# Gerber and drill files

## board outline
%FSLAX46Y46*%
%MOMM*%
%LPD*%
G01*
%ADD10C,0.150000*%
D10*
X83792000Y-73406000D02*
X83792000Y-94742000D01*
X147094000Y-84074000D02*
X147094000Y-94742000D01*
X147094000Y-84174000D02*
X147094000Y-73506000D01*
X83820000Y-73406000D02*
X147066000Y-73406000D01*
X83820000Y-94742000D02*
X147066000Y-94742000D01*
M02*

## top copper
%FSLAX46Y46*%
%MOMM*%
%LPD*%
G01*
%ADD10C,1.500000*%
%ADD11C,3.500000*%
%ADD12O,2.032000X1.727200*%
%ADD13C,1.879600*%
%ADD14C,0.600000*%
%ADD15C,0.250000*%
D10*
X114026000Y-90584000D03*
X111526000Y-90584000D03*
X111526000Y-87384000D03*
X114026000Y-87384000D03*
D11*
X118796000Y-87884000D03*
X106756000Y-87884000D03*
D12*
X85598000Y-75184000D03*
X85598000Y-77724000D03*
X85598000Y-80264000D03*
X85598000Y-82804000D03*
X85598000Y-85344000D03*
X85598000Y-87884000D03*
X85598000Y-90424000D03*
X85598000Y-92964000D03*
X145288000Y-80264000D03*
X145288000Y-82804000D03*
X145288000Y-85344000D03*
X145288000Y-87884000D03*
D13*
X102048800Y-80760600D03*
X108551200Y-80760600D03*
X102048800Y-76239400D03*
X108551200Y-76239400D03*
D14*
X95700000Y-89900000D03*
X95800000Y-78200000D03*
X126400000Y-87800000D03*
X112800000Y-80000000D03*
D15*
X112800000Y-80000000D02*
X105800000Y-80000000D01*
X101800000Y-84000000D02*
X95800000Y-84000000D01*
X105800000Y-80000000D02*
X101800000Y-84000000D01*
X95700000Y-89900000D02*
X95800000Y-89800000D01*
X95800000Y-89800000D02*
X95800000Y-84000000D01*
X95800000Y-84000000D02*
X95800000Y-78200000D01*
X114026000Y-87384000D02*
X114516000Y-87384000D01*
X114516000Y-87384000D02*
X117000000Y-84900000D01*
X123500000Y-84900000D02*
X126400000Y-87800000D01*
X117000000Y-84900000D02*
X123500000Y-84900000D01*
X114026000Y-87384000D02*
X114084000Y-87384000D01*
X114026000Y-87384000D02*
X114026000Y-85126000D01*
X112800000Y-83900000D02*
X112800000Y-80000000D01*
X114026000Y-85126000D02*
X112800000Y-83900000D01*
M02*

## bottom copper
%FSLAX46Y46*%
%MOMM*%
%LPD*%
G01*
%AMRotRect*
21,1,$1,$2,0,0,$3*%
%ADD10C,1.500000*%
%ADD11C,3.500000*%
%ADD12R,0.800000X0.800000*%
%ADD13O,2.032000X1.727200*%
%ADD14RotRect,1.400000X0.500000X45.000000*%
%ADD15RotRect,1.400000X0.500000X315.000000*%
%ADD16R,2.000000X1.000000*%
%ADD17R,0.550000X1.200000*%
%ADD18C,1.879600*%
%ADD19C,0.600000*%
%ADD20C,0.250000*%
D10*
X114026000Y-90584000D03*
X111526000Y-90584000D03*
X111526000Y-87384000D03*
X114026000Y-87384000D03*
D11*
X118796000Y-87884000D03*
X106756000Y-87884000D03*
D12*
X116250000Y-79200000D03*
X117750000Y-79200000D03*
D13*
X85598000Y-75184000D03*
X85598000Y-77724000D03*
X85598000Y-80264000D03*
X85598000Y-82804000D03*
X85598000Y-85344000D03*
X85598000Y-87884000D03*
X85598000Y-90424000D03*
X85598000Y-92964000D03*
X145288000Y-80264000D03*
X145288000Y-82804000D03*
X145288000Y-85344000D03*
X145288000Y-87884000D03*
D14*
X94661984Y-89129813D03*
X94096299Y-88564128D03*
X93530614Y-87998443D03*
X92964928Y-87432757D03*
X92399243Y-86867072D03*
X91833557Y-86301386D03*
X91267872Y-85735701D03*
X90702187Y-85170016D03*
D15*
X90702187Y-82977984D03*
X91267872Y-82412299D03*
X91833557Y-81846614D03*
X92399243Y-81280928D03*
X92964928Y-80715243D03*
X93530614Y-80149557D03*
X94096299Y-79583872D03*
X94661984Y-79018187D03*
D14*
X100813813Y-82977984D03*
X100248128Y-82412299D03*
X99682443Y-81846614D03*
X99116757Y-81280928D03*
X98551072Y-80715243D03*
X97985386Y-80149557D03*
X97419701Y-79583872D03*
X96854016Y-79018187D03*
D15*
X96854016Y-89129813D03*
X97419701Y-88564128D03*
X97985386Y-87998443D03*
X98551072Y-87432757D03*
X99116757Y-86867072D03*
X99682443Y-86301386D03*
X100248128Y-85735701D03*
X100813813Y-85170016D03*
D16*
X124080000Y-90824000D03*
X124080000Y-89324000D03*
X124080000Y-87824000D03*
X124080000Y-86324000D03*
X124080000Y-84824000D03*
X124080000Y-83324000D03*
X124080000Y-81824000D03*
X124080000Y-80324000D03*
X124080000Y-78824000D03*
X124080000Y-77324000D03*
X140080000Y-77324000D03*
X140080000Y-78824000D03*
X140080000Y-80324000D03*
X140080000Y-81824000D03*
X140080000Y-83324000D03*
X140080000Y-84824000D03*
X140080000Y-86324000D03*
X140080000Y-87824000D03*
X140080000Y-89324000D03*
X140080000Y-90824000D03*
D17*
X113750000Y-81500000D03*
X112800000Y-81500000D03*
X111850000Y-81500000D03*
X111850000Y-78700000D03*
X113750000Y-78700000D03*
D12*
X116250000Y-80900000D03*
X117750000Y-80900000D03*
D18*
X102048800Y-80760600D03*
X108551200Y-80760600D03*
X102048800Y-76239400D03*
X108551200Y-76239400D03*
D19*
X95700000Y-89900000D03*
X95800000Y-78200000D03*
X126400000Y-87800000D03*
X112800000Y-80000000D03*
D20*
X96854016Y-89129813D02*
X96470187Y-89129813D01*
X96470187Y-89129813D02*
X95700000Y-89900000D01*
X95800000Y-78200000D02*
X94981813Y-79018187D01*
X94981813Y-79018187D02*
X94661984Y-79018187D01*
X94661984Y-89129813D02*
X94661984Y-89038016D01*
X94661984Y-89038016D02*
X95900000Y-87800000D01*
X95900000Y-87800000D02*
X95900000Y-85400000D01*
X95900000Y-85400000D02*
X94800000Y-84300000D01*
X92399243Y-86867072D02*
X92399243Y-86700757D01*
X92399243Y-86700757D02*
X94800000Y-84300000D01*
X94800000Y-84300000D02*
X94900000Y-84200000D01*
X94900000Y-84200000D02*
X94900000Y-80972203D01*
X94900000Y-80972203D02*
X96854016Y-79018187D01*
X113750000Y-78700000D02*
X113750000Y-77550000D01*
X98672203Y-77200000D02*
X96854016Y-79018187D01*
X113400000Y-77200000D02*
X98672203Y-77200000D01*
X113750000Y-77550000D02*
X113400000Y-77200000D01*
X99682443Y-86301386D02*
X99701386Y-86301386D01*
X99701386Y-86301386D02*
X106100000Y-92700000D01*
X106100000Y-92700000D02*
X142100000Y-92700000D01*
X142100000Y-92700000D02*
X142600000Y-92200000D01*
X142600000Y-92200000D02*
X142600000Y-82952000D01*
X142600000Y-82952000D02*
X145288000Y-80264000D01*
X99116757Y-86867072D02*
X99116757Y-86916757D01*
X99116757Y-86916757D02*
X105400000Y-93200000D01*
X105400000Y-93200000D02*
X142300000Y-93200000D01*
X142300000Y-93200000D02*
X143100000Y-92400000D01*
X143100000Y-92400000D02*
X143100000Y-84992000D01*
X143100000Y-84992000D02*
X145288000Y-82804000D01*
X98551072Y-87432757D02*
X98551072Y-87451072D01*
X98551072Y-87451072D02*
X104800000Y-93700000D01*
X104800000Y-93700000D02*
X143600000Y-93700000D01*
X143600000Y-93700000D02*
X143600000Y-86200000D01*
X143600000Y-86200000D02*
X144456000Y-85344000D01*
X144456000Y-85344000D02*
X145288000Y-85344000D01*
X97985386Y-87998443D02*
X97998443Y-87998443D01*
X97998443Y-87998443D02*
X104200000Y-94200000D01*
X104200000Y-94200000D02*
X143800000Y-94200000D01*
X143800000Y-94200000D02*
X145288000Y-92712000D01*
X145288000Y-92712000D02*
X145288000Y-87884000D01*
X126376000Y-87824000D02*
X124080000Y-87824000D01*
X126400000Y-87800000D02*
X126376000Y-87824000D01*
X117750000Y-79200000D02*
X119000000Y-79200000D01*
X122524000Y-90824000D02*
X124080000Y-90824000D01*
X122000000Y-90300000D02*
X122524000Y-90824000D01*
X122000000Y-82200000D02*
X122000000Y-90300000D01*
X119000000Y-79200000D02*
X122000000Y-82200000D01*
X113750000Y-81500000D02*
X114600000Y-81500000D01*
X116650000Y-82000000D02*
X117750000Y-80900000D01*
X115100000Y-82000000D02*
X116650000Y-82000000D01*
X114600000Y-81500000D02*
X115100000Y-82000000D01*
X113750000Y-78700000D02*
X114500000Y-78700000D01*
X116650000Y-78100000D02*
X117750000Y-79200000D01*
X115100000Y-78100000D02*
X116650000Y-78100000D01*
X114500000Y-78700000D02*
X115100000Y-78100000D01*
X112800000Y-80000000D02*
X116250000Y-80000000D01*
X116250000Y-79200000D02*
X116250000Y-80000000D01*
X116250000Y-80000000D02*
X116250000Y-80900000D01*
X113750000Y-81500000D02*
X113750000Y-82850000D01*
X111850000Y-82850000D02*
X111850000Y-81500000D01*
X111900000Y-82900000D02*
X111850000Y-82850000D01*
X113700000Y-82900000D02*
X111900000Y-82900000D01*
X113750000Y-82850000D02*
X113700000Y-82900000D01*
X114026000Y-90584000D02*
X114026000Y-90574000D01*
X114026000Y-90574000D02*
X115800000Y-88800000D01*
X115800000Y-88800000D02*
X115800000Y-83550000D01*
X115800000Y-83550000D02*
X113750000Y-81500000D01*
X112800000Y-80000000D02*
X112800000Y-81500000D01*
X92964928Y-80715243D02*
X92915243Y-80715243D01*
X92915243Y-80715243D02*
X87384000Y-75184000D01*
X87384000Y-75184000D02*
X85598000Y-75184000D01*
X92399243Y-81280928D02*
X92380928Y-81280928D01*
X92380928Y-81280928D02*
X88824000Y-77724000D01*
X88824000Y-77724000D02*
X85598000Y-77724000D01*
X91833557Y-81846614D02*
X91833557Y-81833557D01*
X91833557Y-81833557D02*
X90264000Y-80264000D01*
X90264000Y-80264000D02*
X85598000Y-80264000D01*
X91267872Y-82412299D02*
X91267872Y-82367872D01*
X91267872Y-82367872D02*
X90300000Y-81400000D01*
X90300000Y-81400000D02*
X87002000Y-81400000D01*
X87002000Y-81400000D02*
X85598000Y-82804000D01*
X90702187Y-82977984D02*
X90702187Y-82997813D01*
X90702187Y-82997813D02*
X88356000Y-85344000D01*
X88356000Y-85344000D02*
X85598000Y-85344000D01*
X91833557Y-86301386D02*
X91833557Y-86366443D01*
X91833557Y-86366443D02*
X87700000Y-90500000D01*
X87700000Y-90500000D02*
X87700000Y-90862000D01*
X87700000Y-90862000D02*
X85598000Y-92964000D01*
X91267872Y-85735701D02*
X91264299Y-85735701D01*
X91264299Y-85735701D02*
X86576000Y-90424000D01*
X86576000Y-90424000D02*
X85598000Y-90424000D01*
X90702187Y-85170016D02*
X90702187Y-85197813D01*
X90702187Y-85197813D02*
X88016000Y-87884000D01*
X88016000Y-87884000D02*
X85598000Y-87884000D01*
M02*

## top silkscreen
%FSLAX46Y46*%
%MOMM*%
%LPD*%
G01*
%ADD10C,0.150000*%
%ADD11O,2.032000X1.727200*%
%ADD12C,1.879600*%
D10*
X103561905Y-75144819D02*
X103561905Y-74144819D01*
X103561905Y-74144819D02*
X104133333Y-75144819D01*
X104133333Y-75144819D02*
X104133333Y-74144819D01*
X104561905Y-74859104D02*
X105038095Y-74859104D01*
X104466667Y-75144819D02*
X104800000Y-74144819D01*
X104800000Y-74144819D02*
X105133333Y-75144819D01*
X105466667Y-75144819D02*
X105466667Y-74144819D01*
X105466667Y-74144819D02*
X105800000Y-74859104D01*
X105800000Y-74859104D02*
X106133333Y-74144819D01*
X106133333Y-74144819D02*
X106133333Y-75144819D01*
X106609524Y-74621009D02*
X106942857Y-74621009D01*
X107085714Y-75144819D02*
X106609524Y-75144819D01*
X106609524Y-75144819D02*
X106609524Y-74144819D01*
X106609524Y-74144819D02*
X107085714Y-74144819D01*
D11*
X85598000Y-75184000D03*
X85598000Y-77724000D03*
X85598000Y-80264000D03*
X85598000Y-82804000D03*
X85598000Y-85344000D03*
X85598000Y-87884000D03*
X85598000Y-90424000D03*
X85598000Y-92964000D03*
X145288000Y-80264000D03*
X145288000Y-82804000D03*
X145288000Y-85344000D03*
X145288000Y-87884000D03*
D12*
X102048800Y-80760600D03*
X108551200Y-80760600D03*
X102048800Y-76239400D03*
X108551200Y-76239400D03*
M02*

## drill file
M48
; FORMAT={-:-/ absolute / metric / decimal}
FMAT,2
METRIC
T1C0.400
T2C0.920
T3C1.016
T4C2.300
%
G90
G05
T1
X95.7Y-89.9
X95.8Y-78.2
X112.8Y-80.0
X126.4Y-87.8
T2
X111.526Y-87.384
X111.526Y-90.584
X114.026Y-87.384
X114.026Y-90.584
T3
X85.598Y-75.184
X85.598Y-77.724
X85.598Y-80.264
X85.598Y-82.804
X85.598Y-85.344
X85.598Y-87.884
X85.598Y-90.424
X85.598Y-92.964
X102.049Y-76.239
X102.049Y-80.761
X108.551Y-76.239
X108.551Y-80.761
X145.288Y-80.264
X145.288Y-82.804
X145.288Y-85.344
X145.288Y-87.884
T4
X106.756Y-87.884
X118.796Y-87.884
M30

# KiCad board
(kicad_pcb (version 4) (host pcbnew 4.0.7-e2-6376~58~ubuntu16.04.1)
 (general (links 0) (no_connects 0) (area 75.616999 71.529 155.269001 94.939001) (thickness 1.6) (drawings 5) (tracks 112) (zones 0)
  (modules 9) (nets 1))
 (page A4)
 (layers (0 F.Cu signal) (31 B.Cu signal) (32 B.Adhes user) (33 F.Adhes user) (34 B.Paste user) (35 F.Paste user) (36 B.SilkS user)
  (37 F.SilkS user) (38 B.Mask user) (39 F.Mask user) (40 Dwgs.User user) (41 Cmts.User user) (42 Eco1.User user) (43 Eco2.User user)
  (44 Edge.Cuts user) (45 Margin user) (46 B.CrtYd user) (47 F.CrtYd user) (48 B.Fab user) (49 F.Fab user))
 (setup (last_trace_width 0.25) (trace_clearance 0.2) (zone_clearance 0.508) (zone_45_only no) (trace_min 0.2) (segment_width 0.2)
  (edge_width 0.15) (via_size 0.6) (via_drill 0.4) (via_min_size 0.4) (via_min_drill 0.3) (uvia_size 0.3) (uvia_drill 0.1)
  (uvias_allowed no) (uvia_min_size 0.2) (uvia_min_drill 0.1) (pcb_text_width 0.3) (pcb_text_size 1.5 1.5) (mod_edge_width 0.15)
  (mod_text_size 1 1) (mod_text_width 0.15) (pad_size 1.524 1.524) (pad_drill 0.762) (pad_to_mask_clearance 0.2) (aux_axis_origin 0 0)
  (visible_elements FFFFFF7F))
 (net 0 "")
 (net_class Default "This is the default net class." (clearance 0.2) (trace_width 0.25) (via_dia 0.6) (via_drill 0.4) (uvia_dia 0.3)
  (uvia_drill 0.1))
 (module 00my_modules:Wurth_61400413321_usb (layer B.Cu) (at 112.776 87.884)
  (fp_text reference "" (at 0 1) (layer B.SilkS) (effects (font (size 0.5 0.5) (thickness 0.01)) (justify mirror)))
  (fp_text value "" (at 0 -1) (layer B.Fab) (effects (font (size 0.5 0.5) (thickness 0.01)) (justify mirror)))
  (pad V thru_hole circle (at 1.25 2.7) (size 1.5 1.5) (drill 0.92) (layers *.Cu *.Mask B.SilkS))
  (pad - thru_hole circle (at -1.25 2.7) (size 1.5 1.5) (drill 0.92) (layers *.Cu *.Mask B.SilkS))
  (pad + thru_hole circle (at -1.25 -0.5) (size 1.5 1.5) (drill 0.92) (layers *.Cu *.Mask B.SilkS))
  (pad G thru_hole circle (at 1.25 -0.5) (size 1.5 1.5) (drill 0.92) (layers *.Cu *.Mask B.SilkS))
  (pad X thru_hole circle (at 6.02 0) (size 3.5 3.5) (drill 2.3) (layers *.Cu *.Mask B.SilkS))
  (pad X thru_hole circle (at -6.02 0) (size 3.5 3.5) (drill 2.3) (layers *.Cu *.Mask B.SilkS)))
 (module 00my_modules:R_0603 (layer B.Cu) (at 117 79.2)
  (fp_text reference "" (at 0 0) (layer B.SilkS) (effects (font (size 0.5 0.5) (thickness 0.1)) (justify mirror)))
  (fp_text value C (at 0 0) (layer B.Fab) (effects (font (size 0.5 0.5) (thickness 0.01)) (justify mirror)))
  (pad 1 smd rect (at -0.75 0) (size 0.8 0.8) (layers B.Cu B.Paste B.Mask))
  (pad 2 smd rect (at 0.75 0) (size 0.8 0.8) (layers B.Cu B.Paste B.Mask)))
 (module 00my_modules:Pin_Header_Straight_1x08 (layer F.Cu) (at 85.598 75.184)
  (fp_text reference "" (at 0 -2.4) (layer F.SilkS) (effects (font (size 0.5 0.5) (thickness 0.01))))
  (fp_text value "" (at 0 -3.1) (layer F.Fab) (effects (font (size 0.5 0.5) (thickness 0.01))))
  (pad 1 thru_hole oval (at 0 0) (size 2.032 1.7272) (drill 1.016) (layers *.Cu *.Mask F.SilkS))
  (pad 2 thru_hole oval (at 0 2.54) (size 2.032 1.7272) (drill 1.016) (layers *.Cu *.Mask F.SilkS))
  (pad 3 thru_hole oval (at 0 5.08) (size 2.032 1.7272) (drill 1.016) (layers *.Cu *.Mask F.SilkS))
  (pad 4 thru_hole oval (at 0 7.62) (size 2.032 1.7272) (drill 1.016) (layers *.Cu *.Mask F.SilkS))
  (pad 5 thru_hole oval (at 0 10.16) (size 2.032 1.7272) (drill 1.016) (layers *.Cu *.Mask F.SilkS))
  (pad 6 thru_hole oval (at 0 12.7) (size 2.032 1.7272) (drill 1.016) (layers *.Cu *.Mask F.SilkS))
  (pad 7 thru_hole oval (at 0 15.24) (size 2.032 1.7272) (drill 1.016) (layers *.Cu *.Mask F.SilkS))
  (pad 8 thru_hole oval (at 0 17.78) (size 2.032 1.7272) (drill 1.016) (layers *.Cu *.Mask F.SilkS)))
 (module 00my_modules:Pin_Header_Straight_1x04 (layer F.Cu) (at 145.288 80.264)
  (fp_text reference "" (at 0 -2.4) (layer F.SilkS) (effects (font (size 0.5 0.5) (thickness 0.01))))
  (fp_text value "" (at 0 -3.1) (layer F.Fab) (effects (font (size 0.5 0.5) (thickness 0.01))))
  (pad 1 thru_hole oval (at 0 0) (size 2.032 1.7272) (drill 1.016) (layers *.Cu *.Mask F.SilkS))
  (pad 2 thru_hole oval (at 0 2.54) (size 2.032 1.7272) (drill 1.016) (layers *.Cu *.Mask F.SilkS))
  (pad 3 thru_hole oval (at 0 5.08) (size 2.032 1.7272) (drill 1.016) (layers *.Cu *.Mask F.SilkS))
  (pad 4 thru_hole oval (at 0 7.62) (size 2.032 1.7272) (drill 1.016) (layers *.Cu *.Mask F.SilkS)))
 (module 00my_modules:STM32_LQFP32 (layer B.Cu) (at 95.758 84.074 45)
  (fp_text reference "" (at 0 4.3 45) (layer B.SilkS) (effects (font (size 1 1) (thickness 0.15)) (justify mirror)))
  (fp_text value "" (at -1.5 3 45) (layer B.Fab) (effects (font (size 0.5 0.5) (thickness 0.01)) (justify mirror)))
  (pad 3.3 smd rect (at -4.35 2.8 45) (size 1.4 0.5) (layers B.Cu B.Paste B.Mask))
  (pad PF0 smd rect (at -4.35 2 45) (size 1.4 0.5) (layers B.Cu B.Paste B.Mask))
  (pad PF1 smd rect (at -4.35 1.2 45) (size 1.4 0.5) (layers B.Cu B.Paste B.Mask))
  (pad RST smd rect (at -4.35 0.4 45) (size 1.4 0.5) (layers B.Cu B.Paste B.Mask))
  (pad 3.3 smd rect (at -4.35 -0.4 45) (size 1.4 0.5) (layers B.Cu B.Paste B.Mask))
  (pad PA0 smd rect (at -4.35 -1.2 45) (size 1.4 0.5) (layers B.Cu B.Paste B.Mask))
  (pad PA1 smd rect (at -4.35 -2 45) (size 1.4 0.5) (layers B.Cu B.Paste B.Mask))
  (pad PA2 smd rect (at -4.35 -2.8 45) (size 1.4 0.5) (layers B.Cu B.Paste B.Mask))
  (pad PA3 smd rect (at -2.8 -4.35 315) (size 1.4 0.5) (layers B.Cu B.Paste B.Mask))
  (pad PA4 smd rect (at -2 -4.35 315) (size 1.4 0.5) (layers B.Cu B.Paste B.Mask))
  (pad PA5 smd rect (at -1.2 -4.35 315) (size 1.4 0.5) (layers B.Cu B.Paste B.Mask))
  (pad PA6 smd rect (at -0.4 -4.35 315) (size 1.4 0.5) (layers B.Cu B.Paste B.Mask))
  (pad PA7 smd rect (at 0.4 -4.35 315) (size 1.4 0.5) (layers B.Cu B.Paste B.Mask))
  (pad PB0 smd rect (at 1.2 -4.35 315) (size 1.4 0.5) (layers B.Cu B.Paste B.Mask))
  (pad PB1 smd rect (at 2 -4.35 315) (size 1.4 0.5) (layers B.Cu B.Paste B.Mask))
  (pad GND smd rect (at 2.8 -4.35 315) (size 1.4 0.5) (layers B.Cu B.Paste B.Mask))
  (pad PA14 smd rect (at 4.35 2.8 45) (size 1.4 0.5) (layers B.Cu B.Paste B.Mask))
  (pad PA13 smd rect (at 4.35 2 45) (size 1.4 0.5) (layers B.Cu B.Paste B.Mask))
  (pad PA12 smd rect (at 4.35 1.2 45) (size 1.4 0.5) (layers B.Cu B.Paste B.Mask))
  (pad PA11 smd rect (at 4.35 0.4 45) (size 1.4 0.5) (layers B.Cu B.Paste B.Mask))
  (pad PA10 smd rect (at 4.35 -0.4 45) (size 1.4 0.5) (layers B.Cu B.Paste B.Mask))
  (pad PA9 smd rect (at 4.35 -1.2 45) (size 1.4 0.5) (layers B.Cu B.Paste B.Mask))
  (pad PA8 smd rect (at 4.35 -2 45) (size 1.4 0.5) (layers B.Cu B.Paste B.Mask))
  (pad 3.3 smd rect (at 4.35 -2.8 45) (size 1.4 0.5) (layers B.Cu B.Paste B.Mask))
  (pad GND smd rect (at -2.8 4.35 315) (size 1.4 0.5) (layers B.Cu B.Paste B.Mask))
  (pad BOOT smd rect (at -2 4.35 315) (size 1.4 0.5) (layers B.Cu B.Paste B.Mask))
  (pad PB7 smd rect (at -1.2 4.35 315) (size 1.4 0.5) (layers B.Cu B.Paste B.Mask))
  (pad PB6 smd rect (at -0.4 4.35 315) (size 1.4 0.5) (layers B.Cu B.Paste B.Mask))
  (pad PB5 smd rect (at 0.4 4.35 315) (size 1.4 0.5) (layers B.Cu B.Paste B.Mask))
  (pad PB4 smd rect (at 1.2 4.35 315) (size 1.4 0.5) (layers B.Cu B.Paste B.Mask))
  (pad PB3 smd rect (at 2 4.35 315) (size 1.4 0.5) (layers B.Cu B.Paste B.Mask))
  (pad PA15 smd rect (at 2.8 4.35 315) (size 1.4 0.5) (layers B.Cu B.Paste B.Mask)))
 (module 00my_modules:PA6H (layer B.Cu) (at 132.08 84.074)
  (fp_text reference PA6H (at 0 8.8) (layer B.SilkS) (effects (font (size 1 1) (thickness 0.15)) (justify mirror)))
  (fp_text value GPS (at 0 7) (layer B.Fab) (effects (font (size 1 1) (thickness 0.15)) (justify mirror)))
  (pad VCC smd rect (at -8 6.75) (size 2 1) (layers B.Cu B.Paste B.Mask))
  (pad 2 smd rect (at -8 5.25) (size 2 1) (layers B.Cu B.Paste B.Mask))
  (pad GND smd rect (at -8 3.75) (size 2 1) (layers B.Cu B.Paste B.Mask))
  (pad 4 smd rect (at -8 2.25) (size 2 1) (layers B.Cu B.Paste B.Mask))
  (pad 5 smd rect (at -8 0.75) (size 2 1) (layers B.Cu B.Paste B.Mask))
  (pad 6 smd rect (at -8 -0.75) (size 2 1) (layers B.Cu B.Paste B.Mask))
  (pad 7 smd rect (at -8 -2.25) (size 2 1) (layers B.Cu B.Paste B.Mask))
  (pad 8 smd rect (at -8 -3.75) (size 2 1) (layers B.Cu B.Paste B.Mask))
  (pad TX smd rect (at -8 -5.25) (size 2 1) (layers B.Cu B.Paste B.Mask))
  (pad RX smd rect (at -8 -6.75) (size 2 1) (layers B.Cu B.Paste B.Mask))
  (pad 11 smd rect (at 8 -6.75) (size 2 1) (layers B.Cu B.Paste B.Mask))
  (pad 12 smd rect (at 8 -5.25) (size 2 1) (layers B.Cu B.Paste B.Mask))
  (pad 13 smd rect (at 8 -3.75) (size 2 1) (layers B.Cu B.Paste B.Mask))
  (pad 14 smd rect (at 8 -2.25) (size 2 1) (layers B.Cu B.Paste B.Mask))
  (pad 15 smd rect (at 8 -0.75) (size 2 1) (layers B.Cu B.Paste B.Mask))
  (pad 16 smd rect (at 8 0.75) (size 2 1) (layers B.Cu B.Paste B.Mask))
  (pad 17 smd rect (at 8 2.25) (size 2 1) (layers B.Cu B.Paste B.Mask))
  (pad 18 smd rect (at 8 3.75) (size 2 1) (layers B.Cu B.Paste B.Mask))
  (pad 19 smd rect (at 8 5.25) (size 2 1) (layers B.Cu B.Paste B.Mask))
  (pad 20 smd rect (at 8 6.75) (size 2 1) (layers B.Cu B.Paste B.Mask)))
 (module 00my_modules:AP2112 (layer B.Cu) (at 112.8 80.1 90)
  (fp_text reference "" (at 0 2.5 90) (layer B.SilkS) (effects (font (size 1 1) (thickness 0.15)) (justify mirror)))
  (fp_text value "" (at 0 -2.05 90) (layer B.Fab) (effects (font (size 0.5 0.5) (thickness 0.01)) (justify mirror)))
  (pad VIN smd rect (at -1.4 0.95 90) (size 1.2 0.55) (layers B.Cu B.Paste B.Mask))
  (pad GND smd rect (at -1.4 0 90) (size 1.2 0.55) (layers B.Cu B.Paste B.Mask))
  (pad EN smd rect (at -1.4 -0.95 90) (size 1.2 0.55) (layers B.Cu B.Paste B.Mask))
  (pad NC smd rect (at 1.4 -0.95 90) (size 1.2 0.55) (layers B.Cu B.Paste B.Mask))
  (pad VOUT smd rect (at 1.4 0.95 90) (size 1.2 0.55) (layers B.Cu B.Paste B.Mask)))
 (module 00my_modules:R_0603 (layer B.Cu) (at 117 80.9)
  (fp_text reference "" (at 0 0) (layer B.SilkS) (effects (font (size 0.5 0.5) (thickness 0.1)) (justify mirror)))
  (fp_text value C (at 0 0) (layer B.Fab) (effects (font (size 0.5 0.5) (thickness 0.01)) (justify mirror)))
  (pad 1 smd rect (at -0.75 0) (size 0.8 0.8) (layers B.Cu B.Paste B.Mask))
  (pad 2 smd rect (at 0.75 0) (size 0.8 0.8) (layers B.Cu B.Paste B.Mask)))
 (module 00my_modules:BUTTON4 (layer F.Cu) (at 105.3 78.5)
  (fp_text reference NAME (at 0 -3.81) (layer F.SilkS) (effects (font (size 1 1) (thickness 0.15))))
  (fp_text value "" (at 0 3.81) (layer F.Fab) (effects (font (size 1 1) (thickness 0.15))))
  (pad 1 thru_hole circle (at -3.2512 2.2606) (size 1.8796 1.8796) (drill 1.016) (layers *.Cu *.Mask F.SilkS))
  (pad 2 thru_hole circle (at 3.2512 2.2606) (size 1.8796 1.8796) (drill 1.016) (layers *.Cu *.Mask F.SilkS))
  (pad 3 thru_hole circle (at -3.2512 -2.2606) (size 1.8796 1.8796) (drill 1.016) (layers *.Cu *.Mask F.SilkS))
  (pad 4 thru_hole circle (at 3.2512 -2.2606) (size 1.8796 1.8796) (drill 1.016) (layers *.Cu *.Mask F.SilkS)))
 (gr_line (start 83.792 73.406) (end 83.792 94.742) (angle 90) (layer Edge.Cuts) (width 0.15))
 (gr_line (start 147.094 84.074) (end 147.094 94.742) (angle 90) (layer Edge.Cuts) (width 0.15))
 (gr_line (start 147.094 84.174) (end 147.094 73.506) (angle 90) (layer Edge.Cuts) (width 0.15))
 (gr_line (start 83.82 73.406) (end 147.066 73.406) (angle 90) (layer Edge.Cuts) (width 0.15))
 (gr_line (start 83.82 94.742) (end 147.066 94.742) (angle 90) (layer Edge.Cuts) (width 0.15))
 (segment (start 112.8 80) (end 105.8 80) (width 0.25) (layer F.Cu) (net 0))
 (segment (start 101.8 84) (end 95.8 84) (width 0.25) (layer F.Cu) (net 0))
 (segment (start 105.8 80) (end 101.8 84) (width 0.25) (layer F.Cu) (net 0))
 (segment (start 96.854016 89.129813) (end 96.470187 89.129813) (width 0.25) (layer B.Cu) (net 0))
 (segment (start 96.470187 89.129813) (end 95.7 89.9) (width 0.25) (layer B.Cu) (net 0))
 (via (at 95.7 89.9) (size 0.6) (drill 0.4) (layers F.Cu B.Cu) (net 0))
 (segment (start 95.7 89.9) (end 95.8 89.8) (width 0.25) (layer F.Cu) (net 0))
 (segment (start 95.8 89.8) (end 95.8 84) (width 0.25) (layer F.Cu) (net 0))
 (segment (start 95.8 78.2) (end 94.981813 79.018187) (width 0.25) (layer B.Cu) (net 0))
 (segment (start 95.8 84) (end 95.8 78.2) (width 0.25) (layer F.Cu) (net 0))
 (via (at 95.8 78.2) (size 0.6) (drill 0.4) (layers F.Cu B.Cu) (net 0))
 (segment (start 94.981813 79.018187) (end 94.661984 79.018187) (width 0.25) (layer B.Cu) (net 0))
 (segment (start 94.661984 89.129813) (end 94.661984 89.038016) (width 0.25) (layer B.Cu) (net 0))
 (segment (start 94.661984 89.038016) (end 95.9 87.8) (width 0.25) (layer B.Cu) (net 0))
 (segment (start 95.9 87.8) (end 95.9 85.4) (width 0.25) (layer B.Cu) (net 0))
 (segment (start 95.9 85.4) (end 94.8 84.3) (width 0.25) (layer B.Cu) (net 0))
 (segment (start 92.399243 86.867072) (end 92.399243 86.700757) (width 0.25) (layer B.Cu) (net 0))
 (segment (start 92.399243 86.700757) (end 94.8 84.3) (width 0.25) (layer B.Cu) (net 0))
 (segment (start 94.8 84.3) (end 94.9 84.2) (width 0.25) (layer B.Cu) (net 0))
 (segment (start 94.9 84.2) (end 94.9 80.972203) (width 0.25) (layer B.Cu) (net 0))
 (segment (start 94.9 80.972203) (end 96.854016 79.018187) (width 0.25) (layer B.Cu) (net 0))
 (segment (start 113.75 78.7) (end 113.75 77.55) (width 0.25) (layer B.Cu) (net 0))
 (segment (start 98.672203 77.2) (end 96.854016 79.018187) (width 0.25) (layer B.Cu) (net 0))
 (segment (start 113.4 77.2) (end 98.672203 77.2) (width 0.25) (layer B.Cu) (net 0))
 (segment (start 113.75 77.55) (end 113.4 77.2) (width 0.25) (layer B.Cu) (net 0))
 (segment (start 99.682443 86.301386) (end 99.701386 86.301386) (width 0.25) (layer B.Cu) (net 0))
 (segment (start 99.701386 86.301386) (end 106.1 92.7) (width 0.25) (layer B.Cu) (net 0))
 (segment (start 106.1 92.7) (end 142.1 92.7) (width 0.25) (layer B.Cu) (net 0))
 (segment (start 142.1 92.7) (end 142.6 92.2) (width 0.25) (layer B.Cu) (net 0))
 (segment (start 142.6 92.2) (end 142.6 82.952) (width 0.25) (layer B.Cu) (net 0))
 (segment (start 142.6 82.952) (end 145.288 80.264) (width 0.25) (layer B.Cu) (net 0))
 (segment (start 99.116757 86.867072) (end 99.116757 86.916757) (width 0.25) (layer B.Cu) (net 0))
 (segment (start 99.116757 86.916757) (end 105.4 93.2) (width 0.25) (layer B.Cu) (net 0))
 (segment (start 105.4 93.2) (end 142.3 93.2) (width 0.25) (layer B.Cu) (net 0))
 (segment (start 142.3 93.2) (end 143.1 92.4) (width 0.25) (layer B.Cu) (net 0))
 (segment (start 143.1 92.4) (end 143.1 84.992) (width 0.25) (layer B.Cu) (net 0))
 (segment (start 143.1 84.992) (end 145.288 82.804) (width 0.25) (layer B.Cu) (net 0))
 (segment (start 98.551072 87.432757) (end 98.551072 87.451072) (width 0.25) (layer B.Cu) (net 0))
 (segment (start 98.551072 87.451072) (end 104.8 93.7) (width 0.25) (layer B.Cu) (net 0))
 (segment (start 104.8 93.7) (end 143.6 93.7) (width 0.25) (layer B.Cu) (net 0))
 (segment (start 143.6 93.7) (end 143.6 86.2) (width 0.25) (layer B.Cu) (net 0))
 (segment (start 143.6 86.2) (end 144.456 85.344) (width 0.25) (layer B.Cu) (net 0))
 (segment (start 144.456 85.344) (end 145.288 85.344) (width 0.25) (layer B.Cu) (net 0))
 (segment (start 97.985386 87.998443) (end 97.998443 87.998443) (width 0.25) (layer B.Cu) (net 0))
 (segment (start 97.998443 87.998443) (end 104.2 94.2) (width 0.25) (layer B.Cu) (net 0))
 (segment (start 104.2 94.2) (end 143.8 94.2) (width 0.25) (layer B.Cu) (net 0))
 (segment (start 143.8 94.2) (end 145.288 92.712) (width 0.25) (layer B.Cu) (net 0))
 (segment (start 145.288 92.712) (end 145.288 87.884) (width 0.25) (layer B.Cu) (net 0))
 (segment (start 114.026 87.384) (end 114.516 87.384) (width 0.25) (layer F.Cu) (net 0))
 (segment (start 114.516 87.384) (end 117 84.9) (width 0.25) (layer F.Cu) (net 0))
 (segment (start 126.376 87.824) (end 124.08 87.824) (width 0.25) (layer B.Cu) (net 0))
 (segment (start 126.4 87.8) (end 126.376 87.824) (width 0.25) (layer B.Cu) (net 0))
 (via (at 126.4 87.8) (size 0.6) (drill 0.4) (layers F.Cu B.Cu) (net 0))
 (segment (start 123.5 84.9) (end 126.4 87.8) (width 0.25) (layer F.Cu) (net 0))
 (segment (start 117 84.9) (end 123.5 84.9) (width 0.25) (layer F.Cu) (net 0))
 (segment (start 117.75 79.2) (end 119 79.2) (width 0.25) (layer B.Cu) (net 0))
 (segment (start 122.524 90.824) (end 124.08 90.824) (width 0.25) (layer B.Cu) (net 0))
 (segment (start 122 90.3) (end 122.524 90.824) (width 0.25) (layer B.Cu) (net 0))
 (segment (start 122 82.2) (end 122 90.3) (width 0.25) (layer B.Cu) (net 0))
 (segment (start 119 79.2) (end 122 82.2) (width 0.25) (layer B.Cu) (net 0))
 (segment (start 113.75 81.5) (end 114.6 81.5) (width 0.25) (layer B.Cu) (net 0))
 (segment (start 116.65 82) (end 117.75 80.9) (width 0.25) (layer B.Cu) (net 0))
 (segment (start 115.1 82) (end 116.65 82) (width 0.25) (layer B.Cu) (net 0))
 (segment (start 114.6 81.5) (end 115.1 82) (width 0.25) (layer B.Cu) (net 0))
 (segment (start 113.75 78.7) (end 114.5 78.7) (width 0.25) (layer B.Cu) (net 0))
 (segment (start 116.65 78.1) (end 117.75 79.2) (width 0.25) (layer B.Cu) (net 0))
 (segment (start 115.1 78.1) (end 116.65 78.1) (width 0.25) (layer B.Cu) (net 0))
 (segment (start 114.5 78.7) (end 115.1 78.1) (width 0.25) (layer B.Cu) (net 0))
 (segment (start 112.8 80) (end 116.25 80) (width 0.25) (layer B.Cu) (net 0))
 (segment (start 116.25 79.2) (end 116.25 80) (width 0.25) (layer B.Cu) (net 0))
 (segment (start 116.25 80) (end 116.25 80.9) (width 0.25) (layer B.Cu) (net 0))
 (segment (start 114.026 87.384) (end 114.084 87.384) (width 0.25) (layer F.Cu) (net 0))
 (segment (start 113.75 81.5) (end 113.75 82.85) (width 0.25) (layer B.Cu) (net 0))
 (segment (start 111.85 82.85) (end 111.85 81.5) (width 0.25) (layer B.Cu) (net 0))
 (segment (start 111.9 82.9) (end 111.85 82.85) (width 0.25) (layer B.Cu) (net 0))
 (segment (start 113.7 82.9) (end 111.9 82.9) (width 0.25) (layer B.Cu) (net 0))
 (segment (start 113.75 82.85) (end 113.7 82.9) (width 0.25) (layer B.Cu) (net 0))
 (segment (start 114.026 90.584) (end 114.026 90.574) (width 0.25) (layer B.Cu) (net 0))
 (segment (start 114.026 90.574) (end 115.8 88.8) (width 0.25) (layer B.Cu) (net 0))
 (segment (start 115.8 88.8) (end 115.8 83.55) (width 0.25) (layer B.Cu) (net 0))
 (segment (start 115.8 83.55) (end 113.75 81.5) (width 0.25) (layer B.Cu) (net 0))
 (segment (start 114.026 87.384) (end 114.026 85.126) (width 0.25) (layer F.Cu) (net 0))
 (segment (start 112.8 80) (end 112.8 81.5) (width 0.25) (layer B.Cu) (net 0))
 (via (at 112.8 80) (size 0.6) (drill 0.4) (layers F.Cu B.Cu) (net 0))
 (segment (start 112.8 83.9) (end 112.8 80) (width 0.25) (layer F.Cu) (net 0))
 (segment (start 114.026 85.126) (end 112.8 83.9) (width 0.25) (layer F.Cu) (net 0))
 (segment (start 92.964928 80.715243) (end 92.915243 80.715243) (width 0.25) (layer B.Cu) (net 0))
 (segment (start 92.915243 80.715243) (end 87.384 75.184) (width 0.25) (layer B.Cu) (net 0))
 (segment (start 87.384 75.184) (end 85.598 75.184) (width 0.25) (layer B.Cu) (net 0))
 (segment (start 92.399243 81.280928) (end 92.380928 81.280928) (width 0.25) (layer B.Cu) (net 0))
 (segment (start 92.380928 81.280928) (end 88.824 77.724) (width 0.25) (layer B.Cu) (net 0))
 (segment (start 88.824 77.724) (end 85.598 77.724) (width 0.25) (layer B.Cu) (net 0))
 (segment (start 91.833557 81.846614) (end 91.833557 81.833557) (width 0.25) (layer B.Cu) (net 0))
 (segment (start 91.833557 81.833557) (end 90.264 80.264) (width 0.25) (layer B.Cu) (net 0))
 (segment (start 90.264 80.264) (end 85.598 80.264) (width 0.25) (layer B.Cu) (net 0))
 (segment (start 91.267872 82.412299) (end 91.267872 82.367872) (width 0.25) (layer B.Cu) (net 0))
 (segment (start 91.267872 82.367872) (end 90.3 81.4) (width 0.25) (layer B.Cu) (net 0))
 (segment (start 90.3 81.4) (end 87.002 81.4) (width 0.25) (layer B.Cu) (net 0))
 (segment (start 87.002 81.4) (end 85.598 82.804) (width 0.25) (layer B.Cu) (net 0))
 (segment (start 90.702187 82.977984) (end 90.702187 82.997813) (width 0.25) (layer B.Cu) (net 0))
 (segment (start 90.702187 82.997813) (end 88.356 85.344) (width 0.25) (layer B.Cu) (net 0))
 (segment (start 88.356 85.344) (end 85.598 85.344) (width 0.25) (layer B.Cu) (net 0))
 (segment (start 91.833557 86.301386) (end 91.833557 86.366443) (width 0.25) (layer B.Cu) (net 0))
 (segment (start 91.833557 86.366443) (end 87.7 90.5) (width 0.25) (layer B.Cu) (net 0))
 (segment (start 87.7 90.5) (end 87.7 90.862) (width 0.25) (layer B.Cu) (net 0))
 (segment (start 87.7 90.862) (end 85.598 92.964) (width 0.25) (layer B.Cu) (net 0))
 (segment (start 91.267872 85.735701) (end 91.264299 85.735701) (width 0.25) (layer B.Cu) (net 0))
 (segment (start 91.264299 85.735701) (end 86.576 90.424) (width 0.25) (layer B.Cu) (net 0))
 (segment (start 86.576 90.424) (end 85.598 90.424) (width 0.25) (layer B.Cu) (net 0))
 (segment (start 90.702187 85.170016) (end 90.702187 85.197813) (width 0.25) (layer B.Cu) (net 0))
 (segment (start 90.702187 85.197813) (end 88.016 87.884) (width 0.25) (layer B.Cu) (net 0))
 (segment (start 88.016 87.884) (end 85.598 87.884) (width 0.25) (layer B.Cu) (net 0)))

